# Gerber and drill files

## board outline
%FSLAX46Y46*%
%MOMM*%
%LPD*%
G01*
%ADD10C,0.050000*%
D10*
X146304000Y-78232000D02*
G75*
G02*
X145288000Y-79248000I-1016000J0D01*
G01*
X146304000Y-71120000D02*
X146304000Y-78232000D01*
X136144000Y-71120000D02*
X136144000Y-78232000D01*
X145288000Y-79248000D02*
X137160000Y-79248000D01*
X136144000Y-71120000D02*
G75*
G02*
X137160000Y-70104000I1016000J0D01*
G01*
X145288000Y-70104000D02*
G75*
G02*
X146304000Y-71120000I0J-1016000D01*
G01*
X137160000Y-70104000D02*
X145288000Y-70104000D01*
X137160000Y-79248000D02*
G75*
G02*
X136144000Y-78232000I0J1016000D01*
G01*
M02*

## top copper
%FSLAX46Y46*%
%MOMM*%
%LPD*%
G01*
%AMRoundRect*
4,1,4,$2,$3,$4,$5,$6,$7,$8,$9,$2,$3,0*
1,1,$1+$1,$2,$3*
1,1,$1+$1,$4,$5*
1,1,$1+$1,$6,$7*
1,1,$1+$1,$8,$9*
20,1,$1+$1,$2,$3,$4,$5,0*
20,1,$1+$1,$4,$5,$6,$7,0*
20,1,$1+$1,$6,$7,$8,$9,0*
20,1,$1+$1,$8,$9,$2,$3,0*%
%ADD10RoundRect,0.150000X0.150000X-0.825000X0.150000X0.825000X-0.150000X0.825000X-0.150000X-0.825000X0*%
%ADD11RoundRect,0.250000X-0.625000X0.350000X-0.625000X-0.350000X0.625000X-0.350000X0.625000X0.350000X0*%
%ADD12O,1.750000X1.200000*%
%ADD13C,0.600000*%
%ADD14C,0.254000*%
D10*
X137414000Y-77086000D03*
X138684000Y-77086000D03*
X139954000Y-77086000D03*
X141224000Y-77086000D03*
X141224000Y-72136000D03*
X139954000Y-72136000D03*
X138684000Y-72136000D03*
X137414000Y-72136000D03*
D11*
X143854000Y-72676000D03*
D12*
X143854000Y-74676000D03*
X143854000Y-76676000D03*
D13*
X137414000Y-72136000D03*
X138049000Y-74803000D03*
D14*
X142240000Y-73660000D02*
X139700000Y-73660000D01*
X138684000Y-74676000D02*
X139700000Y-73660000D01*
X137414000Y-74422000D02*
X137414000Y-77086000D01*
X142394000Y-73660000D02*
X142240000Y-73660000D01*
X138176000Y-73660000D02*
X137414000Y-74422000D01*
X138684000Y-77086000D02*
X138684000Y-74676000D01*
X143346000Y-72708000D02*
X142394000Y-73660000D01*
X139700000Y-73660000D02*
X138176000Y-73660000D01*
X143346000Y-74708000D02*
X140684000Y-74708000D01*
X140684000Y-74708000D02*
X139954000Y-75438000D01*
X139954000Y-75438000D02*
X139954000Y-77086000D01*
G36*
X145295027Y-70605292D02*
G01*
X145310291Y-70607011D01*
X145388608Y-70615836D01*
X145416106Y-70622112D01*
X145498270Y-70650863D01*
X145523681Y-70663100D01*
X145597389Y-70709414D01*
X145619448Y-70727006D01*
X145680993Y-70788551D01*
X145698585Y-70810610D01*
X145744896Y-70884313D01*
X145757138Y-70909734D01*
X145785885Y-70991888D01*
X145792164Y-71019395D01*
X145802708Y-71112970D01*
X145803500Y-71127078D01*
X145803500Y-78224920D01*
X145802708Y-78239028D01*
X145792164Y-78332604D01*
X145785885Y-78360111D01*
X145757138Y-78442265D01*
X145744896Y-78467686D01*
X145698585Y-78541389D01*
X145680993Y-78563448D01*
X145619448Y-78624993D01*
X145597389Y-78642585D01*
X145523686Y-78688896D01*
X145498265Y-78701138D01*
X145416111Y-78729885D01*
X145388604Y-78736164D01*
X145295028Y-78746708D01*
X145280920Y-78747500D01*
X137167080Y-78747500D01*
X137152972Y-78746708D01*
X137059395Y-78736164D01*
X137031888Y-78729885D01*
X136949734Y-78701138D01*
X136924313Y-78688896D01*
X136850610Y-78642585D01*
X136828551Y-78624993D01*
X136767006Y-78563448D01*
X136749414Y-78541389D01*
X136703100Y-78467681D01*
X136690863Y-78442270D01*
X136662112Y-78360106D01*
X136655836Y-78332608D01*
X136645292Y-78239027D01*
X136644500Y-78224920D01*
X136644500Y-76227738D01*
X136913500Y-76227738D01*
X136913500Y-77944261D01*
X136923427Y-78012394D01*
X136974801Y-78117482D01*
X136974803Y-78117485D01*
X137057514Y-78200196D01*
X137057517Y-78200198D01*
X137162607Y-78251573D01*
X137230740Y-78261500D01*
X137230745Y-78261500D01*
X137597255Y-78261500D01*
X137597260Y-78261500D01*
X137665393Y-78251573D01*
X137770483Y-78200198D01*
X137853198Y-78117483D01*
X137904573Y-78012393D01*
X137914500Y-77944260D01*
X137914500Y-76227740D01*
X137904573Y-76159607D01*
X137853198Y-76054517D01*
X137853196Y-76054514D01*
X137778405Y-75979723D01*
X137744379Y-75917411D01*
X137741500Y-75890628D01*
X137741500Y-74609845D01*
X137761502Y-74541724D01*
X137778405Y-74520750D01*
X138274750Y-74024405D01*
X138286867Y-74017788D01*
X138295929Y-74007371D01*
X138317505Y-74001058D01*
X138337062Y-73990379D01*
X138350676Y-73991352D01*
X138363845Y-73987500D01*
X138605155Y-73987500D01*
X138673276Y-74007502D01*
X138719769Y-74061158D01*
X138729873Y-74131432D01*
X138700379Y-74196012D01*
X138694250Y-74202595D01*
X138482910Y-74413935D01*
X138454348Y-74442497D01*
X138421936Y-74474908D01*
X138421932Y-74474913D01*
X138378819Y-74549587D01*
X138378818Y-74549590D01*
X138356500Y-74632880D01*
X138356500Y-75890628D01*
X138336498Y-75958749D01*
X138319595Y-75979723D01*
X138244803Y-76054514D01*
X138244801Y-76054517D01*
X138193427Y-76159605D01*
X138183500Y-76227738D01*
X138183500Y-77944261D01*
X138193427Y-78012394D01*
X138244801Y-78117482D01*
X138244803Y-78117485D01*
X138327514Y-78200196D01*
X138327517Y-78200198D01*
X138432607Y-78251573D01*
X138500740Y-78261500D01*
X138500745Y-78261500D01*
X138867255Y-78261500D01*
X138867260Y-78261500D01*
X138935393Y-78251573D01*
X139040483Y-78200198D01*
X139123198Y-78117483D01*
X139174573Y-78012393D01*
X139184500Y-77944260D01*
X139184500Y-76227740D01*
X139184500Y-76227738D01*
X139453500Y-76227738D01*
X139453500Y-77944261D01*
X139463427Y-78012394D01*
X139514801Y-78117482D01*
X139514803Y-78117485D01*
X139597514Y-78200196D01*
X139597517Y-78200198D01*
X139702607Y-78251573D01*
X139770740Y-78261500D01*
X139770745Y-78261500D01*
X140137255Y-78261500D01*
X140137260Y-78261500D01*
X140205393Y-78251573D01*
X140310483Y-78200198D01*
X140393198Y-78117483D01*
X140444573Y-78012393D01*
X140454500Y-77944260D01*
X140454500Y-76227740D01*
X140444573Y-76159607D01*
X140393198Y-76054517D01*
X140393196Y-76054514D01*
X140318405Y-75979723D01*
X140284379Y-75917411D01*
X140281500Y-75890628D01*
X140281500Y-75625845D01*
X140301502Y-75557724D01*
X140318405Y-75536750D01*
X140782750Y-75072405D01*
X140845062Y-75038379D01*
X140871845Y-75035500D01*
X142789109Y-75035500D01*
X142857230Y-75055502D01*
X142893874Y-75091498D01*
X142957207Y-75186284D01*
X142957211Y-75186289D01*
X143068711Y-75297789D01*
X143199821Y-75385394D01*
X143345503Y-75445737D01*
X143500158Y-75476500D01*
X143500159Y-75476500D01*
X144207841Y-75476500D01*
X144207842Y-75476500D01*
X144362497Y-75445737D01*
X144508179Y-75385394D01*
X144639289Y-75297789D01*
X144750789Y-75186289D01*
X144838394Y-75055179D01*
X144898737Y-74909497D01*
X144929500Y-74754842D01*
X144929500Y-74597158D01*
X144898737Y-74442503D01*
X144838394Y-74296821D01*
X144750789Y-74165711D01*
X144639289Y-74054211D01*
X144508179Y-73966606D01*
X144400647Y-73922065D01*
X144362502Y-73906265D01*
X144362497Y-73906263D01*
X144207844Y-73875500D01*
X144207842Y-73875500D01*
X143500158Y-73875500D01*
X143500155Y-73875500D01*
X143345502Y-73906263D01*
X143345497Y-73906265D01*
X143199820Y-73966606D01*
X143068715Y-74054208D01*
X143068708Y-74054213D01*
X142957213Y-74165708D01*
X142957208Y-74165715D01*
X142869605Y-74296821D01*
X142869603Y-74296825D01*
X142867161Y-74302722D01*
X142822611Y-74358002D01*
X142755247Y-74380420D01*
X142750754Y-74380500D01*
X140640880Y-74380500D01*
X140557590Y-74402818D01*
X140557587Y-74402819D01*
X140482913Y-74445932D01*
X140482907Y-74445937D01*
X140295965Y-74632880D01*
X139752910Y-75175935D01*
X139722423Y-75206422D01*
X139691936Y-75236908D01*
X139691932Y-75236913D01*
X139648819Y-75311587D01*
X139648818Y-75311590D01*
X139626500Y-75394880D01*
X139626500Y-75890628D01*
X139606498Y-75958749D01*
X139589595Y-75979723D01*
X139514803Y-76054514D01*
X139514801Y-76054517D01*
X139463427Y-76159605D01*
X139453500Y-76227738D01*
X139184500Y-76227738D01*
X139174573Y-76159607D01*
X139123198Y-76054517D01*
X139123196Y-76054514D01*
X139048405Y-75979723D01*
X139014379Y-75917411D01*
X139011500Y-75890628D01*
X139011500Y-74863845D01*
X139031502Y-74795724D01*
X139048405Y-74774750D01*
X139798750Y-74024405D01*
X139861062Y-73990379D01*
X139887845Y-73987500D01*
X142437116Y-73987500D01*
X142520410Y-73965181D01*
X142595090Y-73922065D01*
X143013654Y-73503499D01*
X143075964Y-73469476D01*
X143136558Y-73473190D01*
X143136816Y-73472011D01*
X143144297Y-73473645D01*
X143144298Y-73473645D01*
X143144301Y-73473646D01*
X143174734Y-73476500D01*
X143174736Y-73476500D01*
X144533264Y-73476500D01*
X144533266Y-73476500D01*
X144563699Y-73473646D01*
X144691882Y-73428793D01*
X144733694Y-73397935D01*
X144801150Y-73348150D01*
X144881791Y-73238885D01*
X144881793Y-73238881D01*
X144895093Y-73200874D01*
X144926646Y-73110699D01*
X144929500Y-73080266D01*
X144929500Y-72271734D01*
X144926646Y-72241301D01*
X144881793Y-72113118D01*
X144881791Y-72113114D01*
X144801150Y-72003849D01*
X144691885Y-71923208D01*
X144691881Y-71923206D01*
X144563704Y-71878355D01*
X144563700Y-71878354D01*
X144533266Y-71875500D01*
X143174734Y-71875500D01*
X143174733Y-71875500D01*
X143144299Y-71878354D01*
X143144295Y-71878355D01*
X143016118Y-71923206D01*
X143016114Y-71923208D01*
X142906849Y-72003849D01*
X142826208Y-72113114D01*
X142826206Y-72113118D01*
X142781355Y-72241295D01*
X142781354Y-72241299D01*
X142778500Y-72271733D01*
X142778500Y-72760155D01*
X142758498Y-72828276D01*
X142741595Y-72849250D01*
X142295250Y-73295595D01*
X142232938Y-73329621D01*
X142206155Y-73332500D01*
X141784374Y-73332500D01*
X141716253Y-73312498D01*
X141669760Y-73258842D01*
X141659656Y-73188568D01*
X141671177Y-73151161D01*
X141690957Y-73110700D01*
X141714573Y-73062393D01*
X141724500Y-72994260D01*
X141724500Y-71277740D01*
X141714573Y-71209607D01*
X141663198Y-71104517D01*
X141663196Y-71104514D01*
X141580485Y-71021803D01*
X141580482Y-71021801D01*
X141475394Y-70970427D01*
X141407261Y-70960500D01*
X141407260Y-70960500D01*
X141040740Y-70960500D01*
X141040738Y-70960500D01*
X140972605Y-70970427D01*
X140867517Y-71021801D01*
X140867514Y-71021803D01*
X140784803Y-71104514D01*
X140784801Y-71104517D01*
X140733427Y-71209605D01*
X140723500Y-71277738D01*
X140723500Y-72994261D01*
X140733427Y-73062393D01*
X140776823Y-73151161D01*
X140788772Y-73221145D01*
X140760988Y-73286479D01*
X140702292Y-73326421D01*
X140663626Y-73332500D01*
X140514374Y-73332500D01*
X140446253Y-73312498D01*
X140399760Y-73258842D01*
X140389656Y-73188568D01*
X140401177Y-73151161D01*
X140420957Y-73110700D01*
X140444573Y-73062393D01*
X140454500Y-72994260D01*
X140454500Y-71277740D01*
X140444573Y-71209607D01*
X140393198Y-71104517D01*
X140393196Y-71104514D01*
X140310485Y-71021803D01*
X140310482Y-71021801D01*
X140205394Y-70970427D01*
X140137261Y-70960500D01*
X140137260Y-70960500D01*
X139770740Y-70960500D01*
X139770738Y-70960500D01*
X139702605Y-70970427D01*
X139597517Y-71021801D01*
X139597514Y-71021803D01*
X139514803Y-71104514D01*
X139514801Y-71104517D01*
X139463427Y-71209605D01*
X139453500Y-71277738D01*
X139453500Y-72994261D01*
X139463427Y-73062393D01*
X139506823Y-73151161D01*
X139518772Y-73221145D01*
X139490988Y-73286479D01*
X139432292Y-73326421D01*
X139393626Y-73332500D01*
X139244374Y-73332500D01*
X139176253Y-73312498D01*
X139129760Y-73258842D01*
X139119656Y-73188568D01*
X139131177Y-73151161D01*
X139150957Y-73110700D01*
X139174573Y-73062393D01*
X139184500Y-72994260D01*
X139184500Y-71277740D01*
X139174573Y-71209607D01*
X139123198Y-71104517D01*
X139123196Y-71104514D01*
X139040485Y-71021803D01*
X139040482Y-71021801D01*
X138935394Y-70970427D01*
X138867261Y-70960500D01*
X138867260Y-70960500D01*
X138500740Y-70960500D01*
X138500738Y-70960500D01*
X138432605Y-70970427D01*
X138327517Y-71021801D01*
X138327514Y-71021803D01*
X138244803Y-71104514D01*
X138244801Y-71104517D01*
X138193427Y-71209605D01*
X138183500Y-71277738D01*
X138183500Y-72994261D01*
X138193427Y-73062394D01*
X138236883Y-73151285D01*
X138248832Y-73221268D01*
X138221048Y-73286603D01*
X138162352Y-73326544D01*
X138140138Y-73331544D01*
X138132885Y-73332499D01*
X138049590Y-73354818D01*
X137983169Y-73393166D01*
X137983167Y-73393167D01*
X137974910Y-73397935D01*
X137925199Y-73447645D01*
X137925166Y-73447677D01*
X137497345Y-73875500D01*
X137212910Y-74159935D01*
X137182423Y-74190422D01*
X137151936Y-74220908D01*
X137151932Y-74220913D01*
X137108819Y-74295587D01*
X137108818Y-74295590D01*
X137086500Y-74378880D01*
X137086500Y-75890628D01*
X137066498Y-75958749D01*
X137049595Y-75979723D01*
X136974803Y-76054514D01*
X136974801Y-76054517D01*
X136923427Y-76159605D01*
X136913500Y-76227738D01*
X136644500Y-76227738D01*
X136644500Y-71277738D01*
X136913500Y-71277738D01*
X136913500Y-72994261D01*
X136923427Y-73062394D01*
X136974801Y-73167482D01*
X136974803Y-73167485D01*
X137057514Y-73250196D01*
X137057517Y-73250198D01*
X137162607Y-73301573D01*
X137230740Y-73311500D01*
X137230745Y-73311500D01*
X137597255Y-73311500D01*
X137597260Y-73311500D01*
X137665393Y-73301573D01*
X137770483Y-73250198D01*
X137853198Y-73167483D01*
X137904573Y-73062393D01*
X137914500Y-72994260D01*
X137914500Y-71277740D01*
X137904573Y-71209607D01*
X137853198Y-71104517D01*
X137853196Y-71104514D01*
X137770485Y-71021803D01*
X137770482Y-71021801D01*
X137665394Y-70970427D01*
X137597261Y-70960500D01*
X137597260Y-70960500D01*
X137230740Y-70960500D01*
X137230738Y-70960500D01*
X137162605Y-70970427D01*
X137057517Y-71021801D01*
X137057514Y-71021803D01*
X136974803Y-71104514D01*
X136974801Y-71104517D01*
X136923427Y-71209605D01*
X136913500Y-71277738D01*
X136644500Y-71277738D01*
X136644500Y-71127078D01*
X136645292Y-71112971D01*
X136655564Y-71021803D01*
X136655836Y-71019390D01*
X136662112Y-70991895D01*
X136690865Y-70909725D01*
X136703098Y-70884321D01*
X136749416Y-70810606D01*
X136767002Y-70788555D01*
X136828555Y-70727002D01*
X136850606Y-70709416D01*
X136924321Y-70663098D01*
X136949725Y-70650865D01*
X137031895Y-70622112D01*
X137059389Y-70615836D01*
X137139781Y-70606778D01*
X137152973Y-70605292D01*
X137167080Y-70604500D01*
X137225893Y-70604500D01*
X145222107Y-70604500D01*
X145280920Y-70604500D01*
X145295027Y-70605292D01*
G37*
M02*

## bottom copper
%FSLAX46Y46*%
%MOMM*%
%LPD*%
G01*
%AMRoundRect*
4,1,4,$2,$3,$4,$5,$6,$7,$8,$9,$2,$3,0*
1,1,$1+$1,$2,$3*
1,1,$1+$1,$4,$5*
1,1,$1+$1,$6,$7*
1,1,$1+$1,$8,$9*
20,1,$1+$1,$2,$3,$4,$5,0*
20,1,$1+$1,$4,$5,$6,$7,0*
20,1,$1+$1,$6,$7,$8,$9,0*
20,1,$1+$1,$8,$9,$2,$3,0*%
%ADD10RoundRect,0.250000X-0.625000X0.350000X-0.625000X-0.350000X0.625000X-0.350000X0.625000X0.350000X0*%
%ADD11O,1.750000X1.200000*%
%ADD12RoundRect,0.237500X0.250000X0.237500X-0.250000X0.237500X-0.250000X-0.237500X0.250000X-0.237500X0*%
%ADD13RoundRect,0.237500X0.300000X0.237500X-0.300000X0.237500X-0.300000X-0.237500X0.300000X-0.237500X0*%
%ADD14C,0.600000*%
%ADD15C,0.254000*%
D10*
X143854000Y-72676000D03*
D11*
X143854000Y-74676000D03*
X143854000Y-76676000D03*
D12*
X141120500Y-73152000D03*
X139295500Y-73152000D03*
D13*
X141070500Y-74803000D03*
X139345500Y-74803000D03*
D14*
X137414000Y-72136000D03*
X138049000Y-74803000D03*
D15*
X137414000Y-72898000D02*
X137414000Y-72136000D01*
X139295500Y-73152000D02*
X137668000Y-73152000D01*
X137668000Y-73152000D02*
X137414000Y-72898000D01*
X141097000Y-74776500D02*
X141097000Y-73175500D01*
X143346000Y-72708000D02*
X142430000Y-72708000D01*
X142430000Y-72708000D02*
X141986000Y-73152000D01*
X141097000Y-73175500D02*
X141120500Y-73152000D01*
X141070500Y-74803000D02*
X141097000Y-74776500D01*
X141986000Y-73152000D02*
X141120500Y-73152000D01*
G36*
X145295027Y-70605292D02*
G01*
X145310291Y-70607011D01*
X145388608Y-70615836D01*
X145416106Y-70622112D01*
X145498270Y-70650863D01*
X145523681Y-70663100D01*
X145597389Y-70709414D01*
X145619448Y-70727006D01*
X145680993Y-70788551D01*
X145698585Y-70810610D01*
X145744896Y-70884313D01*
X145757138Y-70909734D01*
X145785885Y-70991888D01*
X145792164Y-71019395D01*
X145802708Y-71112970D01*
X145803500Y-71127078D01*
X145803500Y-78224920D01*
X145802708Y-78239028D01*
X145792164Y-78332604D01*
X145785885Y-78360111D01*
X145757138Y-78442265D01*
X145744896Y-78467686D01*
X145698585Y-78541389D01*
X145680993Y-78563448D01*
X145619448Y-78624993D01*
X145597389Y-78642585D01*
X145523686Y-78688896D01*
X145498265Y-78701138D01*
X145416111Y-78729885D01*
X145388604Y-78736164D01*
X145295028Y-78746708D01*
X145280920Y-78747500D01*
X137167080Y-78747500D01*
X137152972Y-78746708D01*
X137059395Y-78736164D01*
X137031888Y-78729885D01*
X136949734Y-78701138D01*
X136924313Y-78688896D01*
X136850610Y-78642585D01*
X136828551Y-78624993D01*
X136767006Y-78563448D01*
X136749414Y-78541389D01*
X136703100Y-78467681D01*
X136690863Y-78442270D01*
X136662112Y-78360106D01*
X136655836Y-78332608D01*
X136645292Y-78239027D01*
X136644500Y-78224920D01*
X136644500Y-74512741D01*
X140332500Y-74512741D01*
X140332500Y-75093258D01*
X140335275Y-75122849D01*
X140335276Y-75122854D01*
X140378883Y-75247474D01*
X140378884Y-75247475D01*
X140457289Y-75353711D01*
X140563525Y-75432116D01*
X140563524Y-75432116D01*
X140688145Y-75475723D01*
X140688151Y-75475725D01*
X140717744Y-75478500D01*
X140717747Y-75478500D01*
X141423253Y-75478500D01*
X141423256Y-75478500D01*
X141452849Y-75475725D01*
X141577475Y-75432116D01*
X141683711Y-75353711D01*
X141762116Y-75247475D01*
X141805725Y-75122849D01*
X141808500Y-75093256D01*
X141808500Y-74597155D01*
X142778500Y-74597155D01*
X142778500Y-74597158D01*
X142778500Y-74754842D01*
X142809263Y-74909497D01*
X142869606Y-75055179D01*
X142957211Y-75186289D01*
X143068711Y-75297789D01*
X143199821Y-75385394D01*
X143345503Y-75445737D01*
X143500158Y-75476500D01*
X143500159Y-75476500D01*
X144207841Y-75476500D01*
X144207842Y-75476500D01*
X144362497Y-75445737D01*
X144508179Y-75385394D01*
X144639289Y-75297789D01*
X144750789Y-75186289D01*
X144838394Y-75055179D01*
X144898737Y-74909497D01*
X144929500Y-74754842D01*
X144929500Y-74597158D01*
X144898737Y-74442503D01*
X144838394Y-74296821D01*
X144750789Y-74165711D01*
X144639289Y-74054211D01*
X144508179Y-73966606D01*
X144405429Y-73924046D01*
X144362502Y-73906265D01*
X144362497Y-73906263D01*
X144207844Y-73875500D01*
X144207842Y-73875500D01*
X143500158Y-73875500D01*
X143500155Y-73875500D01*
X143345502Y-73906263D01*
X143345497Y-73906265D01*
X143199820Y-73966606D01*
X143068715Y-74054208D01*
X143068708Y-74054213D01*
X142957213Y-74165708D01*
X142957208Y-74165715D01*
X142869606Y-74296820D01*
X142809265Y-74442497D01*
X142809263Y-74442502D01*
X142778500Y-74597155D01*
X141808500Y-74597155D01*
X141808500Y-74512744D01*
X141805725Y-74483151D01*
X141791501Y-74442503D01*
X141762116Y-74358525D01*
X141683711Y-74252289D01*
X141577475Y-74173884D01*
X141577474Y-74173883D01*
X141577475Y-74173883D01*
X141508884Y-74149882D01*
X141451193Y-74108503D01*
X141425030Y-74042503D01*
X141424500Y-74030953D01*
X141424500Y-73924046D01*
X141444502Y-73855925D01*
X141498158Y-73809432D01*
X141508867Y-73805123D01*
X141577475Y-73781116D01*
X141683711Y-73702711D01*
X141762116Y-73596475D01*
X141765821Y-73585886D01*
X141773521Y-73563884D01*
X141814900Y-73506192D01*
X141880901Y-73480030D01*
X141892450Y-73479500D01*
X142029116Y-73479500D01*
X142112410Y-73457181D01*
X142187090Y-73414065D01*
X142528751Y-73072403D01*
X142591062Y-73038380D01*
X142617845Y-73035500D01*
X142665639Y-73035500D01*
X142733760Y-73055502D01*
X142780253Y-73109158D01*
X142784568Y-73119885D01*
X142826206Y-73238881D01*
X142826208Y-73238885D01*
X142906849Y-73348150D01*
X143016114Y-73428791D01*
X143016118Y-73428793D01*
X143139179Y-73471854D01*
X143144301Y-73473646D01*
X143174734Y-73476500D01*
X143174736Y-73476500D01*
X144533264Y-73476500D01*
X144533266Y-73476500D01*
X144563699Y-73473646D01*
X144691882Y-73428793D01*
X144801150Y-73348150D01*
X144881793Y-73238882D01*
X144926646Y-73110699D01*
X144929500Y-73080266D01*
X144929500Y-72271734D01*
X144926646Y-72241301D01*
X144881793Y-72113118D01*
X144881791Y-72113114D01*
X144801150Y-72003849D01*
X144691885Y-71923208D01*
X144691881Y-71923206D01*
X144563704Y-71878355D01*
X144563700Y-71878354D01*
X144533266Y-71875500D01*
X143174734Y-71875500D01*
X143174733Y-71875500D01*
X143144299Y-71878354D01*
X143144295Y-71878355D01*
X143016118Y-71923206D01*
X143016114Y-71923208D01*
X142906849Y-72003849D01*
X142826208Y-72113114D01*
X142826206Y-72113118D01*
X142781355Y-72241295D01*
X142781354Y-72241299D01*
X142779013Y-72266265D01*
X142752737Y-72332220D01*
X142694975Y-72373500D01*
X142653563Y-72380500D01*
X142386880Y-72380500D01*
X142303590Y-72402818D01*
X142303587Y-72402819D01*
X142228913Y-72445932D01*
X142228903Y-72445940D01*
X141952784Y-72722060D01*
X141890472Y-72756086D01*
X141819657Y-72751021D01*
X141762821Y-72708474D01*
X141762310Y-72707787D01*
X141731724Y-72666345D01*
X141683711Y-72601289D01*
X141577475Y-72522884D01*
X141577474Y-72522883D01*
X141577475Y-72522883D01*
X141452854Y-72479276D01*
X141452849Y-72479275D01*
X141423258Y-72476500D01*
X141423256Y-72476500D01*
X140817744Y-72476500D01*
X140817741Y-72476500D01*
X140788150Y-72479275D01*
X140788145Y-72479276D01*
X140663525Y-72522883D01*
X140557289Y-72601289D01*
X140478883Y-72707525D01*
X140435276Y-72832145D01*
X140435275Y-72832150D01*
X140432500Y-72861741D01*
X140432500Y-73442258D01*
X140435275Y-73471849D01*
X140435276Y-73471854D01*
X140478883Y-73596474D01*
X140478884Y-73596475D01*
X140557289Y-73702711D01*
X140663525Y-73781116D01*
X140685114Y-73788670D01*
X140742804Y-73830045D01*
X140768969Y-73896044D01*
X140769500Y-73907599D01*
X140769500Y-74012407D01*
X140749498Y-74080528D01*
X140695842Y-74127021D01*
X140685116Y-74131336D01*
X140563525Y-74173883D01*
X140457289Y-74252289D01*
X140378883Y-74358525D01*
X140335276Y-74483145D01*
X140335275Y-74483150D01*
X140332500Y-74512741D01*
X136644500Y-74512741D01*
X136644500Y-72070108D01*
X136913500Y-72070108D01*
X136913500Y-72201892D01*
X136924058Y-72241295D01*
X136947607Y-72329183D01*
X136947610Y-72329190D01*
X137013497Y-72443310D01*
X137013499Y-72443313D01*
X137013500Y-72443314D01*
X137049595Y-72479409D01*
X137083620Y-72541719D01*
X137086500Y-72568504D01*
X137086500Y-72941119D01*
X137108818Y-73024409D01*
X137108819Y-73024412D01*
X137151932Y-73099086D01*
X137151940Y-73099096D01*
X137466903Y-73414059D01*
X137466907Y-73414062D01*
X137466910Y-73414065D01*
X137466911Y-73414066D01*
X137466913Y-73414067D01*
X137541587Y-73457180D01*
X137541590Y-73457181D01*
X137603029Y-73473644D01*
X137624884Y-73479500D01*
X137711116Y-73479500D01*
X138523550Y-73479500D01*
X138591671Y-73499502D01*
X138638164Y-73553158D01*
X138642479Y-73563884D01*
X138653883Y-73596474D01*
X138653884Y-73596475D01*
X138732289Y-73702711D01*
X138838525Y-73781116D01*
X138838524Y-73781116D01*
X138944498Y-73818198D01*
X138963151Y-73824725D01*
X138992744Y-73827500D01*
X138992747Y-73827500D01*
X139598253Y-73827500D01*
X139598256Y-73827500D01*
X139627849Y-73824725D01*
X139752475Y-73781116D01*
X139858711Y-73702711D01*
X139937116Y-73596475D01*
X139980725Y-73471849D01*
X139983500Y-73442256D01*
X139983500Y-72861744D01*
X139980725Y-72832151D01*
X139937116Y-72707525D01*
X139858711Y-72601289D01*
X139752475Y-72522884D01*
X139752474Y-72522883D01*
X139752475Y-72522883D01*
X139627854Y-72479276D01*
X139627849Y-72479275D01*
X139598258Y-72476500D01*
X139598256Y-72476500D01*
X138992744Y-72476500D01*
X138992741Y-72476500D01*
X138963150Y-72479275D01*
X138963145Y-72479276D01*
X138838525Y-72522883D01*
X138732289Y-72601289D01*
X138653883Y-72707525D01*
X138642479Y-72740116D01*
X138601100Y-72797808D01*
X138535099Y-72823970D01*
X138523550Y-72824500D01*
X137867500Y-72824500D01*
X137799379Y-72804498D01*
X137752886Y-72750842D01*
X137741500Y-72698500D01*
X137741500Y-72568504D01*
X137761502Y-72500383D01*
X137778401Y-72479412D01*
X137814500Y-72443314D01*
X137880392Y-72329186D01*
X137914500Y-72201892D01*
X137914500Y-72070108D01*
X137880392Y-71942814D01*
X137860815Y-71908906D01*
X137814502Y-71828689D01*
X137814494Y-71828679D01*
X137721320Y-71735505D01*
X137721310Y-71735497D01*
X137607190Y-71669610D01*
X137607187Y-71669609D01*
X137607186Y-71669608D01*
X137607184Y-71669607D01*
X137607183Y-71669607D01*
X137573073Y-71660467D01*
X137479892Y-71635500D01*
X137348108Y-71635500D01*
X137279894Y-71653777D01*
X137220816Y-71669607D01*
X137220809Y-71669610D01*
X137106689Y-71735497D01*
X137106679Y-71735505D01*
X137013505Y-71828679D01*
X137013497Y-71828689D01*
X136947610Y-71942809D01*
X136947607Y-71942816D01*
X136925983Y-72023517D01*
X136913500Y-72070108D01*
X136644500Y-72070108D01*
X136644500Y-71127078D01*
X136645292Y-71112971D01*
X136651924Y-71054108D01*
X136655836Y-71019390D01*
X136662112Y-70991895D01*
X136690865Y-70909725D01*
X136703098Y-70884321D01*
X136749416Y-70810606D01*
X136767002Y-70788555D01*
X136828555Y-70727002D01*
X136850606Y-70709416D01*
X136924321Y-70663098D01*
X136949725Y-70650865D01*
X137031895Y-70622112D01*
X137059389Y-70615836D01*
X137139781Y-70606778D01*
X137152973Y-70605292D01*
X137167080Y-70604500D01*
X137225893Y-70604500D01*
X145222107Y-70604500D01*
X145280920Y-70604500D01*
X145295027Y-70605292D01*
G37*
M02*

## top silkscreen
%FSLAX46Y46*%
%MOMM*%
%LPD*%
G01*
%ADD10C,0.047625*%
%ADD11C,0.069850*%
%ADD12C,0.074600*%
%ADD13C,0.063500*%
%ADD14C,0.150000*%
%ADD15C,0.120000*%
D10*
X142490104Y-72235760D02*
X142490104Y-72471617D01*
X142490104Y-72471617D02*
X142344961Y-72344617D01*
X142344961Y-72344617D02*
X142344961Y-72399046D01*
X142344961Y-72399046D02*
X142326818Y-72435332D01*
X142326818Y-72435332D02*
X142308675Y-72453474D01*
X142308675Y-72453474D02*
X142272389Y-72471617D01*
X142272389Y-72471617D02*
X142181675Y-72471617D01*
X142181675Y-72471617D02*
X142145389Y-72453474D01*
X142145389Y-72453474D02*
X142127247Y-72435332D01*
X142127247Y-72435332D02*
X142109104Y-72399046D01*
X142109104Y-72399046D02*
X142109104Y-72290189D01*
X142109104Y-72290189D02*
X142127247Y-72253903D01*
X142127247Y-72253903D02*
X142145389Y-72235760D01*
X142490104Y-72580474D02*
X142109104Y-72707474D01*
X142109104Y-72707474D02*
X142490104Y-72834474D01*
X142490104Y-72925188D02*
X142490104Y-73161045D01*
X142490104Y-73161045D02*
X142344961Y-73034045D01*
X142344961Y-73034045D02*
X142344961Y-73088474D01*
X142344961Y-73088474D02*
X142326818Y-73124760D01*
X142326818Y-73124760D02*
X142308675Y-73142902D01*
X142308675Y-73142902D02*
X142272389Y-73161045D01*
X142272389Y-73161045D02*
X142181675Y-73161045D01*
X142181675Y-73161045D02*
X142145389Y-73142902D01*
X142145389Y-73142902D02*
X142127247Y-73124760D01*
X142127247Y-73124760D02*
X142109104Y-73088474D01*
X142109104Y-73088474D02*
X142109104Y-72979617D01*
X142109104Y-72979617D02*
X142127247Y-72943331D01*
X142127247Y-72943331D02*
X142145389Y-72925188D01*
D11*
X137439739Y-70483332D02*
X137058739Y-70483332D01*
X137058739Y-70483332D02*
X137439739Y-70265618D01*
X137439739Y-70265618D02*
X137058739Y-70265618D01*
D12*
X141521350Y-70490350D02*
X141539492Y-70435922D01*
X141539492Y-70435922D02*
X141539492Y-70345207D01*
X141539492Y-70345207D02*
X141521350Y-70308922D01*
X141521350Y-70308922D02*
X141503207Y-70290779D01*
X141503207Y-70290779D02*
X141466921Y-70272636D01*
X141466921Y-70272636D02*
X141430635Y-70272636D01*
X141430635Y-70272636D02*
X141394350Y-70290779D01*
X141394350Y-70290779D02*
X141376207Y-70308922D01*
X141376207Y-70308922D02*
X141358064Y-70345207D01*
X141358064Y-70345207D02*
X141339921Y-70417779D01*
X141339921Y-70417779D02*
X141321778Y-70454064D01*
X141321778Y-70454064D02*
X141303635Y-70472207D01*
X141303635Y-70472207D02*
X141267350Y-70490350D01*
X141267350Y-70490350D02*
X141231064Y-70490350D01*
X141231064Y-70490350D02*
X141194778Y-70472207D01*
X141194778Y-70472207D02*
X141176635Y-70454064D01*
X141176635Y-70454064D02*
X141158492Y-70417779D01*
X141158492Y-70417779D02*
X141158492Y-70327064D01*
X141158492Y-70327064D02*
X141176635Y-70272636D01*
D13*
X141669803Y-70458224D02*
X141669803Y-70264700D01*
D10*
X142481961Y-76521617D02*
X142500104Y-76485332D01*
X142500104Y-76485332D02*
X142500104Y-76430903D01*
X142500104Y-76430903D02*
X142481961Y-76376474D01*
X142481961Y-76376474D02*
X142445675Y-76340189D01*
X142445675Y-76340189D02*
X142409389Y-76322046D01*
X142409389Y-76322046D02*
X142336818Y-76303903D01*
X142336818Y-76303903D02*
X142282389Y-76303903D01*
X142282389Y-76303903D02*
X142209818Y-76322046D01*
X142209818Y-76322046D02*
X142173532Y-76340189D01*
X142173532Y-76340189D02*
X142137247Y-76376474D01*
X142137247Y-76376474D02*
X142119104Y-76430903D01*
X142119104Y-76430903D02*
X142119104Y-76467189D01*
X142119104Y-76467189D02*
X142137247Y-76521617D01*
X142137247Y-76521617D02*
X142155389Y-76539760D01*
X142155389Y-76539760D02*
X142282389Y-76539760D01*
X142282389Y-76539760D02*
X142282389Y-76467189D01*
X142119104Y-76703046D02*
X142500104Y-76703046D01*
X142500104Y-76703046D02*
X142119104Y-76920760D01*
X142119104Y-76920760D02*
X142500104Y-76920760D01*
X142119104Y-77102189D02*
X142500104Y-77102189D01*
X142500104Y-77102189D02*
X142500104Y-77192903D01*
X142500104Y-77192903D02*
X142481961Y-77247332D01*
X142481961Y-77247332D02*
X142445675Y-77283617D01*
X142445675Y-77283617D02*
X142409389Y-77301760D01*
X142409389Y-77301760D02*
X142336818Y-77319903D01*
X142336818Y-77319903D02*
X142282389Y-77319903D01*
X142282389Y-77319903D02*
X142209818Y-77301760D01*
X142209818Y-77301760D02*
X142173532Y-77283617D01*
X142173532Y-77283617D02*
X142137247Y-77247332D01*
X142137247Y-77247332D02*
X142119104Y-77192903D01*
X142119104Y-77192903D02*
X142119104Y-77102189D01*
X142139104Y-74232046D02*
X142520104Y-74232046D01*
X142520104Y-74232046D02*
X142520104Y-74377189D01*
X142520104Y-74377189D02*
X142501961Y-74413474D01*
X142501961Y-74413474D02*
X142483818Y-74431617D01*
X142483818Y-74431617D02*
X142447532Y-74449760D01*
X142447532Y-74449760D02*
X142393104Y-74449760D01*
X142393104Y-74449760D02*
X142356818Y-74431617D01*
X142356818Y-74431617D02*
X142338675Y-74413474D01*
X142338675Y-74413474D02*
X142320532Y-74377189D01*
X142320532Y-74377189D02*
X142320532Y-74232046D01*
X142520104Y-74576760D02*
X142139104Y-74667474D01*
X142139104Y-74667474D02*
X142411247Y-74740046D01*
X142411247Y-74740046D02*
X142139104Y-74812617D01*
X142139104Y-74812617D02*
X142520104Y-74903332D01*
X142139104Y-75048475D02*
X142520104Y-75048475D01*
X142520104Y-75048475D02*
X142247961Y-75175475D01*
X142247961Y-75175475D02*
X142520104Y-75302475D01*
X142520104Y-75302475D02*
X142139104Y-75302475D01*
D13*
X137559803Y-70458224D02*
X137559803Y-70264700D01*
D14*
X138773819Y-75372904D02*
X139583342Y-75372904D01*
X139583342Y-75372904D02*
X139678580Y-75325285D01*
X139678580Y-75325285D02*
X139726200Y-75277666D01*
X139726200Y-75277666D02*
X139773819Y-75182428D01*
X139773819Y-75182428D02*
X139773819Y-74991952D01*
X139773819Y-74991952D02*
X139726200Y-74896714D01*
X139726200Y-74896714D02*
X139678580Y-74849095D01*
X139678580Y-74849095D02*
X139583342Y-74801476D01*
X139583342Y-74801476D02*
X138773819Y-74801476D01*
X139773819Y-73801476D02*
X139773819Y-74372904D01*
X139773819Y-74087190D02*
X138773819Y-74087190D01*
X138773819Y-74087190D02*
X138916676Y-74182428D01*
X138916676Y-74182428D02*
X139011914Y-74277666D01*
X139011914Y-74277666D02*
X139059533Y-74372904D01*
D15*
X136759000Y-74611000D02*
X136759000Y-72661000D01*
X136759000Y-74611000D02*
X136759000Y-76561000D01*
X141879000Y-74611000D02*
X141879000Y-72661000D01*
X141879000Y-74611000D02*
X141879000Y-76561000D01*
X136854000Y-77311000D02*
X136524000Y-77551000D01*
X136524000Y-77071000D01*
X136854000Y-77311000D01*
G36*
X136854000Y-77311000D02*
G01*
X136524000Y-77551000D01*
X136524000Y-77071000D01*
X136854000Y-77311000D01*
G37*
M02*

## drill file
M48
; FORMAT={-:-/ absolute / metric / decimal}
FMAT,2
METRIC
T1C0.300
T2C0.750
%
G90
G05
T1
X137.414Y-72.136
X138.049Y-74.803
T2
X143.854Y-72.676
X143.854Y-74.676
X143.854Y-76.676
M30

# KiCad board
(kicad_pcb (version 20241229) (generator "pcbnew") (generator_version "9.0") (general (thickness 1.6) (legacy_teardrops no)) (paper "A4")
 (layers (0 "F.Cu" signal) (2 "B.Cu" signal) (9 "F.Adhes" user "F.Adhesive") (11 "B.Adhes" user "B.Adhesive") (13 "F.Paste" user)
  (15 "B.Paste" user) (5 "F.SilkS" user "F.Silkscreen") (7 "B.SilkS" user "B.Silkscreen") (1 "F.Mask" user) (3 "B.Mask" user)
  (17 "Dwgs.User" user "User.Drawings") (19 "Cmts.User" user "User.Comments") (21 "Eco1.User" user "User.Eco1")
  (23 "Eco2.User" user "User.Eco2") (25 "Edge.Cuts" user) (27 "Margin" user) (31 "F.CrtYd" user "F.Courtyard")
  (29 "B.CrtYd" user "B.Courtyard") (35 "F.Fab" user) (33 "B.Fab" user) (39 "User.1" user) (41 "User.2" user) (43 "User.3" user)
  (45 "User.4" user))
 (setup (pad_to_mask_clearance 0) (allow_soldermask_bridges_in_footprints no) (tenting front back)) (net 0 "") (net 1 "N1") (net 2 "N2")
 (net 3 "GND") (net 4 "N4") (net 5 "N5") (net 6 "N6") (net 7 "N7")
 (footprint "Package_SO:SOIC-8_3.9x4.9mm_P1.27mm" (layer "F.Cu") (at 139.319 74.611 90)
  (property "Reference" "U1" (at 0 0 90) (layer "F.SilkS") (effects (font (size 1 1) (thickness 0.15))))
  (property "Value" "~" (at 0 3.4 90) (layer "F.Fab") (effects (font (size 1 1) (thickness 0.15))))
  (fp_line (start 0 -2.56) (end 1.95 -2.56) (stroke (width 0.12) (type solid)) (layer "F.SilkS"))
  (fp_line (start 0 -2.56) (end -1.95 -2.56) (stroke (width 0.12) (type solid)) (layer "F.SilkS"))
  (fp_line (start 0 2.56) (end 1.95 2.56) (stroke (width 0.12) (type solid)) (layer "F.SilkS"))
  (fp_line (start 0 2.56) (end -1.95 2.56) (stroke (width 0.12) (type solid)) (layer "F.SilkS"))
  (fp_poly (pts (xy -2.7 -2.465) (xy -2.94 -2.795) (xy -2.46 -2.795)) (stroke (width 0.12) (type solid)) (fill yes) (layer "F.SilkS"))
  (pad "1" smd roundrect (at -2.475 -1.905 90) (size 1.95 0.6) (layers "F.Cu" "F.Mask" "F.Paste") (roundrect_rratio 0.25) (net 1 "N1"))
  (pad "2" smd roundrect (at -2.475 -0.635 90) (size 1.95 0.6) (layers "F.Cu" "F.Mask" "F.Paste") (roundrect_rratio 0.25) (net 1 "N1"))
  (pad "3" smd roundrect (at -2.475 0.635 90) (size 1.95 0.6) (layers "F.Cu" "F.Mask" "F.Paste") (roundrect_rratio 0.25) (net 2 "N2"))
  (pad "4" smd roundrect (at -2.475 1.905 90) (size 1.95 0.6) (layers "F.Cu" "F.Mask" "F.Paste") (roundrect_rratio 0.25) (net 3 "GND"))
  (pad "5" smd roundrect (at 2.475 1.905 90) (size 1.95 0.6) (layers "F.Cu" "F.Mask" "F.Paste") (roundrect_rratio 0.25) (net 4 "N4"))
  (pad "6" smd roundrect (at 2.475 0.635 90) (size 1.95 0.6) (layers "F.Cu" "F.Mask" "F.Paste") (roundrect_rratio 0.25) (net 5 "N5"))
  (pad "7" smd roundrect (at 2.475 -0.635 90) (size 1.95 0.6) (layers "F.Cu" "F.Mask" "F.Paste") (roundrect_rratio 0.25) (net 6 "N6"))
  (pad "8" smd roundrect (at 2.475 -1.905 90) (size 1.95 0.6) (layers "F.Cu" "F.Mask" "F.Paste") (roundrect_rratio 0.25) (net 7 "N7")))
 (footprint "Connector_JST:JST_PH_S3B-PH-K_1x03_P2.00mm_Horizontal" (layer "B.Cu") (at 143.854 72.676 -90)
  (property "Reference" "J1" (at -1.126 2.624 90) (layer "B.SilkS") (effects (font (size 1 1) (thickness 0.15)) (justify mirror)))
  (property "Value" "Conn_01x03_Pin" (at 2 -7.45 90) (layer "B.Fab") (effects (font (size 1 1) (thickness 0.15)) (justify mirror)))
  (pad "1" thru_hole roundrect (at 0 0 270) (size 1.2 1.75) (drill 0.75) (layers "*.Cu" "*.Mask") (remove_unused_layers no)
   (roundrect_rratio 0.208333) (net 1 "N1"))
  (pad "2" thru_hole oval (at 2 0 270) (size 1.2 1.75) (drill 0.75) (layers "*.Cu" "*.Mask") (remove_unused_layers no) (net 2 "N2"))
  (pad "3" thru_hole oval (at 4 0 270) (size 1.2 1.75) (drill 0.75) (layers "*.Cu" "*.Mask") (remove_unused_layers no) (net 3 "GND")))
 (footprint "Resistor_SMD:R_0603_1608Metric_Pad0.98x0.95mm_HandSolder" (layer "B.Cu") (at 140.208 73.152 180)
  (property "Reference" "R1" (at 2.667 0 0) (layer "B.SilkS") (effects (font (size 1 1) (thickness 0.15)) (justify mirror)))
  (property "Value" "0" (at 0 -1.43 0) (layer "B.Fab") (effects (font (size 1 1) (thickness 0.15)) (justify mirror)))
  (pad "1" smd roundrect (at -0.9125 0 180) (size 0.975 0.95) (layers "B.Cu" "B.Mask" "B.Paste") (roundrect_rratio 0.25) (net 1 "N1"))
  (pad "2" smd roundrect (at 0.9125 0 180) (size 0.975 0.95) (layers "B.Cu" "B.Mask" "B.Paste") (roundrect_rratio 0.25) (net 7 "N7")))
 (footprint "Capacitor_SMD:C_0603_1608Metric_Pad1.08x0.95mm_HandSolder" (layer "B.Cu") (at 140.208 74.803 180)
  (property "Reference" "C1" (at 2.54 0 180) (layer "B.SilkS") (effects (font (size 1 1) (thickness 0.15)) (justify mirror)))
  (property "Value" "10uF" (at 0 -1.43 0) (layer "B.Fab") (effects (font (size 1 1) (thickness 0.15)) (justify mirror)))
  (pad "1" smd roundrect (at -0.8625 0 180) (size 1.075 0.95) (layers "B.Cu" "B.Mask" "B.Paste") (roundrect_rratio 0.25) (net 1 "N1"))
  (pad "2" smd roundrect (at 0.8625 0 180) (size 1.075 0.95) (layers "B.Cu" "B.Mask" "B.Paste") (roundrect_rratio 0.25) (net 3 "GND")))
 (gr_arc (start 146.304 78.232) (mid 146.00642 78.95042) (end 145.288 79.248) (stroke (width 0.05) (type default)) (layer "Edge.Cuts"))
 (gr_line (start 146.304 71.12) (end 146.304 78.232) (stroke (width 0.05) (type default)) (layer "Edge.Cuts"))
 (gr_line (start 136.144 71.12) (end 136.144 78.232) (stroke (width 0.05) (type default)) (layer "Edge.Cuts"))
 (gr_line (start 145.288 79.248) (end 137.16 79.248) (stroke (width 0.05) (type default)) (layer "Edge.Cuts"))
 (gr_arc (start 136.144 71.12) (mid 136.44158 70.40158) (end 137.16 70.104) (stroke (width 0.05) (type default)) (layer "Edge.Cuts"))
 (gr_arc (start 145.288 70.104) (mid 146.00642 70.40158) (end 146.304 71.12) (stroke (width 0.05) (type default)) (layer "Edge.Cuts"))
 (gr_line (start 137.16 70.104) (end 145.288 70.104) (stroke (width 0.05) (type default)) (layer "Edge.Cuts"))
 (gr_arc (start 137.16 79.248) (mid 136.44158 78.95042) (end 136.144 78.232) (stroke (width 0.05) (type default)) (layer "Edge.Cuts"))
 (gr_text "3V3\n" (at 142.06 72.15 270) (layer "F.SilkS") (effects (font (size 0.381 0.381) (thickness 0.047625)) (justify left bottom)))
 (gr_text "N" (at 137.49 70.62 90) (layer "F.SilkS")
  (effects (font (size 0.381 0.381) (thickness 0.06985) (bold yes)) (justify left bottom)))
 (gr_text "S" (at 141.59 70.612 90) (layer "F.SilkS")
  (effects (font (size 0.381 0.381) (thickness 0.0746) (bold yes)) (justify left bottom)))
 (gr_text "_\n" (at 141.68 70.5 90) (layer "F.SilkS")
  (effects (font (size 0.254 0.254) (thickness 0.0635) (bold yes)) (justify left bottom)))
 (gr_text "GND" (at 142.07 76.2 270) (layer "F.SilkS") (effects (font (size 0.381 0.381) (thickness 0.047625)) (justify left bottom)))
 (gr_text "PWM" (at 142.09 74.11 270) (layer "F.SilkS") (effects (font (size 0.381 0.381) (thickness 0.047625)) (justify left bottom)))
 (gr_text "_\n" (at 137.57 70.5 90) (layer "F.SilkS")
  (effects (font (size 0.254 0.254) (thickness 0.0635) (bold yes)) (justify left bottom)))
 (via (at 137.414 72.136) (size 0.6) (drill 0.3) (layers "F.Cu" "B.Cu") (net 7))
 (segment (start 137.414 72.898) (end 137.414 72.136) (width 0.254) (layer "B.Cu") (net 7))
 (segment (start 139.2955 73.152) (end 137.668 73.152) (width 0.254) (layer "B.Cu") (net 7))
 (segment (start 137.668 73.152) (end 137.414 72.898) (width 0.254) (layer "B.Cu") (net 7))
 (via (at 138.049 74.803) (size 0.6) (drill 0.3) (layers "F.Cu" "B.Cu") (free yes) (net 3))
 (segment (start 142.24 73.66) (end 139.7 73.66) (width 0.254) (layer "F.Cu") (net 1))
 (segment (start 138.684 74.676) (end 139.7 73.66) (width 0.254) (layer "F.Cu") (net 1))
 (segment (start 137.414 74.422) (end 137.414 77.086) (width 0.254) (layer "F.Cu") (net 1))
 (segment (start 142.394 73.66) (end 142.24 73.66) (width 0.254) (layer "F.Cu") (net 1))
 (segment (start 138.176 73.66) (end 137.414 74.422) (width 0.254) (layer "F.Cu") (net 1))
 (segment (start 138.684 77.086) (end 138.684 74.676) (width 0.254) (layer "F.Cu") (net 1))
 (segment (start 143.346 72.708) (end 142.394 73.66) (width 0.254) (layer "F.Cu") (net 1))
 (segment (start 139.7 73.66) (end 138.176 73.66) (width 0.254) (layer "F.Cu") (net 1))
 (segment (start 141.097 74.7765) (end 141.097 73.1755) (width 0.254) (layer "B.Cu") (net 1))
 (segment (start 143.346 72.708) (end 142.43 72.708) (width 0.254) (layer "B.Cu") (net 1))
 (segment (start 142.43 72.708) (end 141.986 73.152) (width 0.254) (layer "B.Cu") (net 1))
 (segment (start 141.097 73.1755) (end 141.1205 73.152) (width 0.254) (layer "B.Cu") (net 1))
 (segment (start 141.0705 74.803) (end 141.097 74.7765) (width 0.254) (layer "B.Cu") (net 1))
 (segment (start 141.986 73.152) (end 141.1205 73.152) (width 0.254) (layer "B.Cu") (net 1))
 (segment (start 143.346 74.708) (end 140.684 74.708) (width 0.254) (layer "F.Cu") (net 2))
 (segment (start 140.684 74.708) (end 139.954 75.438) (width 0.254) (layer "F.Cu") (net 2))
 (segment (start 139.954 75.438) (end 139.954 77.086) (width 0.254) (layer "F.Cu") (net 2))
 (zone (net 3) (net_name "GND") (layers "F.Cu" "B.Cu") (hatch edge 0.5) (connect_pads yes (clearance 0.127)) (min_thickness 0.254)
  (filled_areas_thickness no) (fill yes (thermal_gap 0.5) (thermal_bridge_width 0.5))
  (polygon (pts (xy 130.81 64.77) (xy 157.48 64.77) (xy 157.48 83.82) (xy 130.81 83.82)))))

